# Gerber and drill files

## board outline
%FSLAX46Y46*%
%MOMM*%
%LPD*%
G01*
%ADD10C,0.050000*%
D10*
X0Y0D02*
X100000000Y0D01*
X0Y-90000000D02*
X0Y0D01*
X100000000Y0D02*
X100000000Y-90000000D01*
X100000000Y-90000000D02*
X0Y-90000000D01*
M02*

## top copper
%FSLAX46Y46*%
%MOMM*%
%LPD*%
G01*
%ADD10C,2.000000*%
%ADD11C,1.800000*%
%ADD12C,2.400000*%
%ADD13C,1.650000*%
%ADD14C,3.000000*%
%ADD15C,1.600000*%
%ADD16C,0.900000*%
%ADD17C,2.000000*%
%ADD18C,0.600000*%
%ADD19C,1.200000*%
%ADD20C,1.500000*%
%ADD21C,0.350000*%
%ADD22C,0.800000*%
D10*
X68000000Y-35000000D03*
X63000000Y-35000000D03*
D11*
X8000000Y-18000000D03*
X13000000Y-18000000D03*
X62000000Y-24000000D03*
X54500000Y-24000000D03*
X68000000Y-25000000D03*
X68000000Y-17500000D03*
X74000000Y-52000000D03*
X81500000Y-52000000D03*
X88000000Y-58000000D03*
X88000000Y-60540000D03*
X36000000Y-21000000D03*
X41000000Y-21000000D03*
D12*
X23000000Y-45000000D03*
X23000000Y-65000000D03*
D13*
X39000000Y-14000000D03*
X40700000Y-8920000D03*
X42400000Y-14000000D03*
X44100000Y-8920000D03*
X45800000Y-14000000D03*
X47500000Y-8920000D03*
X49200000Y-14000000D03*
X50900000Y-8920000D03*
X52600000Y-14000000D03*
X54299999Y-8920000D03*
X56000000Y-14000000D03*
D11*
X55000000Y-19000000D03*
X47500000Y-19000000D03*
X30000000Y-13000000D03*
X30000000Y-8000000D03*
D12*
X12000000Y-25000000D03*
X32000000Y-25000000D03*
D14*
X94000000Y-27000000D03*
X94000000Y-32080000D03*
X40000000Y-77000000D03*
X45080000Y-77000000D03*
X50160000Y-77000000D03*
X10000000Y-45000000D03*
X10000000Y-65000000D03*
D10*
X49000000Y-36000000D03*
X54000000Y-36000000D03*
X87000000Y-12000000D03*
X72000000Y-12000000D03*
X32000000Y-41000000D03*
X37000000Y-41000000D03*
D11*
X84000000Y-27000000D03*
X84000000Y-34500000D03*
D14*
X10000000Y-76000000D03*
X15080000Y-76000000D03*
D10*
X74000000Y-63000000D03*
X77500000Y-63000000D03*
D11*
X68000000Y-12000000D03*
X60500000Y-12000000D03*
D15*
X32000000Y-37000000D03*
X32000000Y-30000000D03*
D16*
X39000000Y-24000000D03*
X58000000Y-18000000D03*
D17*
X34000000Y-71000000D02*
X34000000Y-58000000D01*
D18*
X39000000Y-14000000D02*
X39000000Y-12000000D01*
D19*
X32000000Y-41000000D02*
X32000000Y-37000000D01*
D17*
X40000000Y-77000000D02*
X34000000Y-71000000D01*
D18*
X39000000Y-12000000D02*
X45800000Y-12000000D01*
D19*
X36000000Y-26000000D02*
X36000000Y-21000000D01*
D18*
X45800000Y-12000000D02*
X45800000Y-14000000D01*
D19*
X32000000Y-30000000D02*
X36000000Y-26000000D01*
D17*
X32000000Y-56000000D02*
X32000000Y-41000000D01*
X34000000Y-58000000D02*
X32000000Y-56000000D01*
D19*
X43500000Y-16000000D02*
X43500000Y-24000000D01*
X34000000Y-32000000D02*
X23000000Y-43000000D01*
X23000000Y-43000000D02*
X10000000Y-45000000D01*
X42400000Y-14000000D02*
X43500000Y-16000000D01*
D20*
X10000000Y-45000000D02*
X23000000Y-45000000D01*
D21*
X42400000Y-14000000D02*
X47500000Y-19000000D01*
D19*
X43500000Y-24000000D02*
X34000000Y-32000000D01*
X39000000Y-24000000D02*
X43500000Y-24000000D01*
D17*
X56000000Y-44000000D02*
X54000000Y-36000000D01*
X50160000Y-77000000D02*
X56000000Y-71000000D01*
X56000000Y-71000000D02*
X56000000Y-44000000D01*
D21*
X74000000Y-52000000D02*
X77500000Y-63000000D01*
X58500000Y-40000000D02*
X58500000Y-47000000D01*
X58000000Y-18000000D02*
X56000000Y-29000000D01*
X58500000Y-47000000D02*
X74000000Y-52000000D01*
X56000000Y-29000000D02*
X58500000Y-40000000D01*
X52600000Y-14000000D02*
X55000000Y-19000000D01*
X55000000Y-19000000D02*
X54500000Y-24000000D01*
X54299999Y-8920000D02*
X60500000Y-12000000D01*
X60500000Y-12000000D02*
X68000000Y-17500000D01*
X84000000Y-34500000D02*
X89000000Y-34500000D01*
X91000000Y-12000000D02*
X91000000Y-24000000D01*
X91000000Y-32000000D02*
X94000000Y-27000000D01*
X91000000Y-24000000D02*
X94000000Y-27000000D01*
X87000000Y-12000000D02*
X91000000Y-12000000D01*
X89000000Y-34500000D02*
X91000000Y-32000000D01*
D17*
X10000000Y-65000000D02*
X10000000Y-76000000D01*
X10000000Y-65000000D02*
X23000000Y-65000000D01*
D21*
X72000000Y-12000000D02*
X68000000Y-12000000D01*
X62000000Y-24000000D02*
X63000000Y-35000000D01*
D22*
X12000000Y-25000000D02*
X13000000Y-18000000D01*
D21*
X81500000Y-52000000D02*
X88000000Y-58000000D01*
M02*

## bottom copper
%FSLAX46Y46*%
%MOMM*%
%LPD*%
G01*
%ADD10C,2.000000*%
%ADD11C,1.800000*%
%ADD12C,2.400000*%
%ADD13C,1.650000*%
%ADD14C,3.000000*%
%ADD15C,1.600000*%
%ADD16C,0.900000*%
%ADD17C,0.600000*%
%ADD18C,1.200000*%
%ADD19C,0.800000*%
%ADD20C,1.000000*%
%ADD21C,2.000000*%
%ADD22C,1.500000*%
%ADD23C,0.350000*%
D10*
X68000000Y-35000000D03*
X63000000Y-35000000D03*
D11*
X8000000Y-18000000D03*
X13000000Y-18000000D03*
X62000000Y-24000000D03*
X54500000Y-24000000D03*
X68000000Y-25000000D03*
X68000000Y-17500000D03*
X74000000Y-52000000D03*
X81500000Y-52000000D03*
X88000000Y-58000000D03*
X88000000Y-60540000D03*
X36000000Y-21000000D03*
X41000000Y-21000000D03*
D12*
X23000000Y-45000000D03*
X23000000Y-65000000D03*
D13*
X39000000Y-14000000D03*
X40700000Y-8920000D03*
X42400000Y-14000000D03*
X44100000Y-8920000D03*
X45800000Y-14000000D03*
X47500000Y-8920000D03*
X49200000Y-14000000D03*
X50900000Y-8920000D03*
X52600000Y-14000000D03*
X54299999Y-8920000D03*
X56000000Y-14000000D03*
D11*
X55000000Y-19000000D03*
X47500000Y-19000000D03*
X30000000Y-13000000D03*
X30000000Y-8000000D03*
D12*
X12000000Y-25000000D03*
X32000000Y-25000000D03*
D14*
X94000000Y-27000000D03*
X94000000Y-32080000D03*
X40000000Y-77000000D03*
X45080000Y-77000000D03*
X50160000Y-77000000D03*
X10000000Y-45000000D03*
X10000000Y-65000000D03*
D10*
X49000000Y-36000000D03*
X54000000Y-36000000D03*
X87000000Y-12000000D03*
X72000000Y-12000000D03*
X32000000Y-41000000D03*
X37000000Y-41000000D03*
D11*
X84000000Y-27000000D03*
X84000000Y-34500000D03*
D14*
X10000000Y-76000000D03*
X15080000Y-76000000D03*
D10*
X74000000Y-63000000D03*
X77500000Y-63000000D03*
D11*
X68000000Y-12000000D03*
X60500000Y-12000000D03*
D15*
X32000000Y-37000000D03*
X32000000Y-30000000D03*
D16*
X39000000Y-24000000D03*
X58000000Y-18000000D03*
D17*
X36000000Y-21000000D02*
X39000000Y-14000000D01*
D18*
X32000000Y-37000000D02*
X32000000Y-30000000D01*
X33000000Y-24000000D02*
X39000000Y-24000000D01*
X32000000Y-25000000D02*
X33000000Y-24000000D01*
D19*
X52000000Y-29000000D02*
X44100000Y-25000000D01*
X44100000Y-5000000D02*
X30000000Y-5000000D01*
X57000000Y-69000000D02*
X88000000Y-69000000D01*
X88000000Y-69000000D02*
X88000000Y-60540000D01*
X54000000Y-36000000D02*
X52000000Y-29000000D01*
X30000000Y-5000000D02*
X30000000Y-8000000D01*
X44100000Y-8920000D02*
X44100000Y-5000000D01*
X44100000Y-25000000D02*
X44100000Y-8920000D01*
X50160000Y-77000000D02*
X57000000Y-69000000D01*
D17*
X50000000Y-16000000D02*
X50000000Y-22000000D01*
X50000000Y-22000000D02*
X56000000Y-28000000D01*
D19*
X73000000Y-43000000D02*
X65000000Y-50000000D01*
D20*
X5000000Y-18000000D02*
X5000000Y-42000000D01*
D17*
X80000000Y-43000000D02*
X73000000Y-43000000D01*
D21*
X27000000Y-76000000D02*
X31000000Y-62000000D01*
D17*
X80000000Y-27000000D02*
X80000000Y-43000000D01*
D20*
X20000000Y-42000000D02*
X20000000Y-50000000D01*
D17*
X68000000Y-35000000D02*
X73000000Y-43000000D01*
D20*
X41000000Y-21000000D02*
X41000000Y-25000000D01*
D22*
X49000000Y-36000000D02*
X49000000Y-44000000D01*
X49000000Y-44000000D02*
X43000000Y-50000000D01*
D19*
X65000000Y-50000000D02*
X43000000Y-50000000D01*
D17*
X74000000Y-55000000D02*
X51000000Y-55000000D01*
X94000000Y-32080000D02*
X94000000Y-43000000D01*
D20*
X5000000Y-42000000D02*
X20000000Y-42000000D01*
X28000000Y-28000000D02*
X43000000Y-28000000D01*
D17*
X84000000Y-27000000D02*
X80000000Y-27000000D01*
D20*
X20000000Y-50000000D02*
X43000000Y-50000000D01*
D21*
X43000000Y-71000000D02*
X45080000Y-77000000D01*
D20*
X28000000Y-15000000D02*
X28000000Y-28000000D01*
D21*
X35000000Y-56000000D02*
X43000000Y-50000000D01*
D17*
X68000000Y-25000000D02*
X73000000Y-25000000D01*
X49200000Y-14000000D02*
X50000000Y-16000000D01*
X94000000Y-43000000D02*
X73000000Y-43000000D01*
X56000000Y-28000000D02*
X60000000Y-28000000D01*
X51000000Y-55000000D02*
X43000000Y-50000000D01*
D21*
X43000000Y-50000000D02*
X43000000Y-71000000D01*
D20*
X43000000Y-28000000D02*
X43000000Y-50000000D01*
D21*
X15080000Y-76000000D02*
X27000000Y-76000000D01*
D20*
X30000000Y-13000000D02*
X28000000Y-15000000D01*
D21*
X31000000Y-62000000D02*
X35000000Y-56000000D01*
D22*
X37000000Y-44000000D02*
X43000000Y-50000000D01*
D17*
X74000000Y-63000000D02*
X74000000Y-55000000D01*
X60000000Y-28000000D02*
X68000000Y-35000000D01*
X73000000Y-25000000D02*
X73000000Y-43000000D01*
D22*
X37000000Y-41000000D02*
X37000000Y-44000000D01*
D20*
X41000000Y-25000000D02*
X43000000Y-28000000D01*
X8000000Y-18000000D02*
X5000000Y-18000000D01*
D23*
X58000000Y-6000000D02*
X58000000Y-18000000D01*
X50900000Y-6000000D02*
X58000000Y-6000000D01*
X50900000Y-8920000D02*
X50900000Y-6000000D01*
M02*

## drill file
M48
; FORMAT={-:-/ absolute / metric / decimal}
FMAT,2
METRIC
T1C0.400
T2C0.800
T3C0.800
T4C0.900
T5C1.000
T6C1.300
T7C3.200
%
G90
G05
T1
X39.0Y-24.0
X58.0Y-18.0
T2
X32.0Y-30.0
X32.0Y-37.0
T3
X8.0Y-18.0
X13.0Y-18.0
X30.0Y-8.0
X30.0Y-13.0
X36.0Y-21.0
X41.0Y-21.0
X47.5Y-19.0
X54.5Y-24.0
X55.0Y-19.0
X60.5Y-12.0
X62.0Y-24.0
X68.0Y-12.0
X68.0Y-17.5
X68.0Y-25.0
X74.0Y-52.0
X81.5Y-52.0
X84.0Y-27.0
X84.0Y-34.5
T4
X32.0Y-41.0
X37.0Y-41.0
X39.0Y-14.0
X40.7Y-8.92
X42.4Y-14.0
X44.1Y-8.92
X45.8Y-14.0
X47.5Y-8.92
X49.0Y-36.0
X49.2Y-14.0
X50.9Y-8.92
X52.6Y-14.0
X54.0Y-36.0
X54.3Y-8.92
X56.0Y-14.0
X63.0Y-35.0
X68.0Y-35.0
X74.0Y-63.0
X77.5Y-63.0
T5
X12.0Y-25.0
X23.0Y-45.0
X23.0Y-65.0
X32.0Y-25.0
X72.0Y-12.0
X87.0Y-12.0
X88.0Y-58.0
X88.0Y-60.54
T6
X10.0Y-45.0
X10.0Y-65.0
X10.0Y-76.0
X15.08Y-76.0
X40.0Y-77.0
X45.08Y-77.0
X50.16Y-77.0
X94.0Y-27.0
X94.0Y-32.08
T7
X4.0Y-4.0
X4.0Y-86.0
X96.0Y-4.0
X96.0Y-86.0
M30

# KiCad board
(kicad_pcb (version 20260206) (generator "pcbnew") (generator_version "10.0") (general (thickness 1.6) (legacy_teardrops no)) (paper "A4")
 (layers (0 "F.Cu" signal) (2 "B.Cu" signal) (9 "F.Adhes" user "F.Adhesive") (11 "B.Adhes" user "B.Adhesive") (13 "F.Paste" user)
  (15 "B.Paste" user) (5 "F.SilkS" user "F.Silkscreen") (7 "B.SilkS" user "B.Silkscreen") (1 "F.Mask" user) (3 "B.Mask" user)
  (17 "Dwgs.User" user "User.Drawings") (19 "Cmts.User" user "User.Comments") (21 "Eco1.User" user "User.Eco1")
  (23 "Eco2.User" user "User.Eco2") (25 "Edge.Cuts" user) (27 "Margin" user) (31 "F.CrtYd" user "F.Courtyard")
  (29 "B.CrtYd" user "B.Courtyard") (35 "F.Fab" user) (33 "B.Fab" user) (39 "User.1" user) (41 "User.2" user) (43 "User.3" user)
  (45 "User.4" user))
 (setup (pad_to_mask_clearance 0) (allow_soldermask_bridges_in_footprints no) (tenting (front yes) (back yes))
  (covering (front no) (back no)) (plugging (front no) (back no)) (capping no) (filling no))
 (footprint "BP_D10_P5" (layer "F.Cu") (at 68 35 180)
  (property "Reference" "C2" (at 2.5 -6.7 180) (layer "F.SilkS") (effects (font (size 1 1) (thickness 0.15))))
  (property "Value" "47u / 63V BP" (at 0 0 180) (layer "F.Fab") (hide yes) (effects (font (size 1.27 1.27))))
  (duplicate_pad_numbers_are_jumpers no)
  (pad "1" thru_hole circle (at 0 0 180) (size 2 2) (drill 0.9) (layers "*.Cu" "*.Mask") (remove_unused_layers no) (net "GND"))
  (pad "2" thru_hole circle (at 5 0 180) (size 2 2) (drill 0.9) (layers "*.Cu" "*.Mask") (remove_unused_layers no) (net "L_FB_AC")))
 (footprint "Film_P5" (layer "F.Cu") (at 8 18)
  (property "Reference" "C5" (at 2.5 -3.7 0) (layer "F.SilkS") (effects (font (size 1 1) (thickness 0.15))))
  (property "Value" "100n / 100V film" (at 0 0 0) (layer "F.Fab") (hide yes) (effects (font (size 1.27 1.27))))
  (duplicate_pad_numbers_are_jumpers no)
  (pad "1" thru_hole circle (at 0 0) (size 1.8 1.8) (drill 0.8) (layers "*.Cu" "*.Mask") (remove_unused_layers no) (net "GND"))
  (pad "2" thru_hole circle (at 5 0) (size 1.8 1.8) (drill 0.8) (layers "*.Cu" "*.Mask") (remove_unused_layers no) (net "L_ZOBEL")))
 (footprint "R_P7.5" (layer "F.Cu") (at 62 24 180)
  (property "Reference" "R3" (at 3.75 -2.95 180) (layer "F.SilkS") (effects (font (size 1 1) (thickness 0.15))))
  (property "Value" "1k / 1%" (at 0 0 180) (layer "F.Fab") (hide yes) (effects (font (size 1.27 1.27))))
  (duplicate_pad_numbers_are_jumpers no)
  (pad "1" thru_hole circle (at 0 0 180) (size 1.8 1.8) (drill 0.8) (layers "*.Cu" "*.Mask") (remove_unused_layers no) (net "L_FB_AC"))
  (pad "2" thru_hole circle (at 7.5 0 180) (size 1.8 1.8) (drill 0.8) (layers "*.Cu" "*.Mask") (remove_unused_layers no) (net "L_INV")))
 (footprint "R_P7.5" (layer "F.Cu") (at 68 25 90)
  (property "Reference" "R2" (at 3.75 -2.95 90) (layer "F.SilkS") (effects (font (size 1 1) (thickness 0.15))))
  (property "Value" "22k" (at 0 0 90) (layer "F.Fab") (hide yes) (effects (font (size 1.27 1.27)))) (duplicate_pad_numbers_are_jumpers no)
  (pad "1" thru_hole circle (at 0 0 90) (size 1.8 1.8) (drill 0.8) (layers "*.Cu" "*.Mask") (remove_unused_layers no) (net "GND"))
  (pad "2" thru_hole circle (at 7.5 0 90) (size 1.8 1.8) (drill 0.8) (layers "*.Cu" "*.Mask") (remove_unused_layers no) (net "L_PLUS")))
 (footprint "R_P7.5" (layer "F.Cu") (at 74 52)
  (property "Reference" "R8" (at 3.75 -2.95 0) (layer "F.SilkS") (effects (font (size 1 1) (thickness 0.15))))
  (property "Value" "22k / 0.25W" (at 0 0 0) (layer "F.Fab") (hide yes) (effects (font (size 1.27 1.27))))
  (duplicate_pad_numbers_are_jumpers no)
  (pad "1" thru_hole circle (at 0 0) (size 1.8 1.8) (drill 0.8) (layers "*.Cu" "*.Mask") (remove_unused_layers no) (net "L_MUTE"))
  (pad "2" thru_hole circle (at 7.5 0) (size 1.8 1.8) (drill 0.8) (layers "*.Cu" "*.Mask") (remove_unused_layers no) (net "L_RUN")))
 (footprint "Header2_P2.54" (layer "F.Cu") (at 88 58 -90)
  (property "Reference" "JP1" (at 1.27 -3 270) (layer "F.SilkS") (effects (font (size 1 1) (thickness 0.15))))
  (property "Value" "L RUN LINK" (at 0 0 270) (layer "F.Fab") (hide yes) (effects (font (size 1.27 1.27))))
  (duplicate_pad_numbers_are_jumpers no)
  (pad "1" thru_hole circle (at 0 0 270) (size 1.8 1.8) (drill 1) (layers "*.Cu" "*.Mask") (remove_unused_layers no) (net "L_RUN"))
  (pad "2" thru_hole circle (at 2.54 0 270) (size 1.8 1.8) (drill 1) (layers "*.Cu" "*.Mask") (remove_unused_layers no) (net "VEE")))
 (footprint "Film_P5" (layer "F.Cu") (at 36 21)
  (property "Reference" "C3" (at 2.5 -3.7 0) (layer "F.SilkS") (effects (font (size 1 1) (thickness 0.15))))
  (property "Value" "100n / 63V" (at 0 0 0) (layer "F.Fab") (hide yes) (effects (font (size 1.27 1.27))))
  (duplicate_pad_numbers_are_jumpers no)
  (pad "1" thru_hole circle (at 0 0) (size 1.8 1.8) (drill 0.8) (layers "*.Cu" "*.Mask") (remove_unused_layers no) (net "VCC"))
  (pad "2" thru_hole circle (at 5 0) (size 1.8 1.8) (drill 0.8) (layers "*.Cu" "*.Mask") (remove_unused_layers no) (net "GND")))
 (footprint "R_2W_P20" (layer "F.Cu") (at 23 45 -90)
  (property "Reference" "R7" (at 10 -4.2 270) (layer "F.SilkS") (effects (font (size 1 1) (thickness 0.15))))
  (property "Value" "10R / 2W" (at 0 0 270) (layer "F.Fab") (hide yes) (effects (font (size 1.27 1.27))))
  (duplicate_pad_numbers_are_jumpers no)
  (pad "1" thru_hole circle (at 0 0 270) (size 2.4 2.4) (drill 1) (layers "*.Cu" "*.Mask") (remove_unused_layers no) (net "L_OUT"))
  (pad "2" thru_hole circle (at 20 0 270) (size 2.4 2.4) (drill 1) (layers "*.Cu" "*.Mask") (remove_unused_layers no) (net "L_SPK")))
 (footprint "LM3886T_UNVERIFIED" (layer "F.Cu") (at 39 14)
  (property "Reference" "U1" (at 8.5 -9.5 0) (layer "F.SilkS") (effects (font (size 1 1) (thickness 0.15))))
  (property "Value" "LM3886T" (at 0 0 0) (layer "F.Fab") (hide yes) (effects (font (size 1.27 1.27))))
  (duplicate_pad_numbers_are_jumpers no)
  (pad "1" thru_hole circle (at 0 0) (size 1.65 1.65) (drill 0.9) (layers "*.Cu" "*.Mask") (remove_unused_layers no) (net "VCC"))
  (pad "2" thru_hole circle (at 1.7 -5.08) (size 1.65 1.65) (drill 0.9) (layers "*.Cu" "*.Mask") (remove_unused_layers no)
   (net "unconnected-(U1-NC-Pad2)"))
  (pad "3" thru_hole circle (at 3.4 0) (size 1.65 1.65) (drill 0.9) (layers "*.Cu" "*.Mask") (remove_unused_layers no) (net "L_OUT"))
  (pad "4" thru_hole circle (at 5.1 -5.08) (size 1.65 1.65) (drill 0.9) (layers "*.Cu" "*.Mask") (remove_unused_layers no) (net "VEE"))
  (pad "5" thru_hole circle (at 6.8 0) (size 1.65 1.65) (drill 0.9) (layers "*.Cu" "*.Mask") (remove_unused_layers no) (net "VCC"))
  (pad "6" thru_hole circle (at 8.5 -5.08) (size 1.65 1.65) (drill 0.9) (layers "*.Cu" "*.Mask") (remove_unused_layers no)
   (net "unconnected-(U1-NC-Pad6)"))
  (pad "7" thru_hole circle (at 10.2 0) (size 1.65 1.65) (drill 0.9) (layers "*.Cu" "*.Mask") (remove_unused_layers no) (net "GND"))
  (pad "8" thru_hole circle (at 11.9 -5.08) (size 1.65 1.65) (drill 0.9) (layers "*.Cu" "*.Mask") (remove_unused_layers no) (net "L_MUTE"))
  (pad "9" thru_hole circle (at 13.6 0) (size 1.65 1.65) (drill 0.9) (layers "*.Cu" "*.Mask") (remove_unused_layers no) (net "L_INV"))
  (pad "10" thru_hole circle (at 15.299999 -5.08) (size 1.65 1.65) (drill 0.9) (layers "*.Cu" "*.Mask") (remove_unused_layers no)
   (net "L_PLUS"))
  (pad "11" thru_hole circle (at 17 0) (size 1.65 1.65) (drill 0.9) (layers "*.Cu" "*.Mask") (remove_unused_layers no)
   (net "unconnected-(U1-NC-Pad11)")))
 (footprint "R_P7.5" (layer "F.Cu") (at 55 19 180)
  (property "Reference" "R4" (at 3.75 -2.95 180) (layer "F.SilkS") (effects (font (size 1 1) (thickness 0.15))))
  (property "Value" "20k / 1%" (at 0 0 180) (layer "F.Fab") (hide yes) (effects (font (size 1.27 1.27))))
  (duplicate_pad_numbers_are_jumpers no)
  (pad "1" thru_hole circle (at 0 0 180) (size 1.8 1.8) (drill 0.8) (layers "*.Cu" "*.Mask") (remove_unused_layers no) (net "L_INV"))
  (pad "2" thru_hole circle (at 7.5 0 180) (size 1.8 1.8) (drill 0.8) (layers "*.Cu" "*.Mask") (remove_unused_layers no) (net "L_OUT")))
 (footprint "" (layer "F.Cu") (at 96 4)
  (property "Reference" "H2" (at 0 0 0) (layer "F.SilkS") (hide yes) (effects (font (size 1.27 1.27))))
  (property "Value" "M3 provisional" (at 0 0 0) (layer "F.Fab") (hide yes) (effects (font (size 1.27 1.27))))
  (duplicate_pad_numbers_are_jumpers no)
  (pad "" np_thru_hole circle (at 0 0) (size 3.2 3.2) (drill 3.2) (layers "*.Cu" "*.Mask")))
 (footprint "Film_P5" (layer "F.Cu") (at 30 13 90)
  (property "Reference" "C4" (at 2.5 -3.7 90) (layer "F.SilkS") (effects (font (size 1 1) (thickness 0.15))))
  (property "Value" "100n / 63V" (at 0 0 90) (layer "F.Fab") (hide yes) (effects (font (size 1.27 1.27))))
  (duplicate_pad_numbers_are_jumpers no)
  (pad "1" thru_hole circle (at 0 0 90) (size 1.8 1.8) (drill 0.8) (layers "*.Cu" "*.Mask") (remove_unused_layers no) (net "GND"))
  (pad "2" thru_hole circle (at 5 0 90) (size 1.8 1.8) (drill 0.8) (layers "*.Cu" "*.Mask") (remove_unused_layers no) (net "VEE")))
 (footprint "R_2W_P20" (layer "F.Cu") (at 12 25)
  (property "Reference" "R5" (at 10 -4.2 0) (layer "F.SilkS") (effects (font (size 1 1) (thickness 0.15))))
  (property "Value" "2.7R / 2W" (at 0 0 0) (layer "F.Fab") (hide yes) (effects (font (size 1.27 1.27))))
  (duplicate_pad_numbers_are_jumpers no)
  (pad "1" thru_hole circle (at 0 0) (size 2.4 2.4) (drill 1) (layers "*.Cu" "*.Mask") (remove_unused_layers no) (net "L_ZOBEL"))
  (pad "2" thru_hole circle (at 20 0) (size 2.4 2.4) (drill 1) (layers "*.Cu" "*.Mask") (remove_unused_layers no) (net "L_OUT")))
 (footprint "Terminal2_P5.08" (layer "F.Cu") (at 94 27 -90)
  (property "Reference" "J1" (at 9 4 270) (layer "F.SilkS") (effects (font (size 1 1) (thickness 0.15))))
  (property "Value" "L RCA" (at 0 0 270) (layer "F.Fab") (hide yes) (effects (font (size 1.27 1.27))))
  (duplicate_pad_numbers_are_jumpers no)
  (pad "1" thru_hole circle (at 0 0 270) (size 3 3) (drill 1.3) (layers "*.Cu" "*.Mask") (remove_unused_layers no) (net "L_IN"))
  (pad "2" thru_hole circle (at 5.08 0 270) (size 3 3) (drill 1.3) (layers "*.Cu" "*.Mask") (remove_unused_layers no) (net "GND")))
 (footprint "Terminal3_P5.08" (layer "F.Cu") (at 40 77)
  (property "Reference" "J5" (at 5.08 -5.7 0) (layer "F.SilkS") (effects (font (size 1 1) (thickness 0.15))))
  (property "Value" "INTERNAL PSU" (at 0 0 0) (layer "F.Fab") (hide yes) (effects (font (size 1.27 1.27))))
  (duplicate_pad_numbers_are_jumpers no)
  (pad "1" thru_hole circle (at 0 0) (size 3 3) (drill 1.3) (layers "*.Cu" "*.Mask") (remove_unused_layers no) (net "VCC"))
  (pad "2" thru_hole circle (at 5.08 0) (size 3 3) (drill 1.3) (layers "*.Cu" "*.Mask") (remove_unused_layers no) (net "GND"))
  (pad "3" thru_hole circle (at 10.16 0) (size 3 3) (drill 1.3) (layers "*.Cu" "*.Mask") (remove_unused_layers no) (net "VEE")))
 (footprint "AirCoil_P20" (layer "F.Cu") (at 10 45 -90)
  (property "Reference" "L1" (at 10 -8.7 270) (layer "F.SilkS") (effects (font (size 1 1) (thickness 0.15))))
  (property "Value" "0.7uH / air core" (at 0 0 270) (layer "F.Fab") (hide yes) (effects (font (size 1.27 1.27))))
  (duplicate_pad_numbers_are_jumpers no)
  (pad "1" thru_hole circle (at 0 0 270) (size 3 3) (drill 1.3) (layers "*.Cu" "*.Mask") (remove_unused_layers no) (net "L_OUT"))
  (pad "2" thru_hole circle (at 20 0 270) (size 3 3) (drill 1.3) (layers "*.Cu" "*.Mask") (remove_unused_layers no) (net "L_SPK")))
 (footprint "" (layer "F.Cu") (at 96 86)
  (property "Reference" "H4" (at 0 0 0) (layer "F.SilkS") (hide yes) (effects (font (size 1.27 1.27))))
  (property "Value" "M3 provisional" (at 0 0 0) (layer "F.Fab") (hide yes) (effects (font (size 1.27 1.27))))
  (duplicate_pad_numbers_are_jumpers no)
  (pad "" np_thru_hole circle (at 0 0) (size 3.2 3.2) (drill 3.2) (layers "*.Cu" "*.Mask")))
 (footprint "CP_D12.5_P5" (layer "F.Cu") (at 49 36)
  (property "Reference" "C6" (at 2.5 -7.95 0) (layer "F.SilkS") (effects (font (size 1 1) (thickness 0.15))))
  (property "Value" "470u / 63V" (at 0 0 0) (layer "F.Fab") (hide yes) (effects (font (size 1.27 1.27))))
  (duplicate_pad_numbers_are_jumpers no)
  (pad "1" thru_hole circle (at 0 0) (size 2 2) (drill 0.9) (layers "*.Cu" "*.Mask") (remove_unused_layers no) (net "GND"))
  (pad "2" thru_hole circle (at 5 0) (size 2 2) (drill 0.9) (layers "*.Cu" "*.Mask") (remove_unused_layers no) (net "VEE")))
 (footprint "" (layer "F.Cu") (at 4 4)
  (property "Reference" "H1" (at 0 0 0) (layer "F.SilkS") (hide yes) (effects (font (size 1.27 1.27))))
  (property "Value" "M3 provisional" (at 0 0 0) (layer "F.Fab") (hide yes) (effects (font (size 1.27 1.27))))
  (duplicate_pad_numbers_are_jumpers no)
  (pad "" np_thru_hole circle (at 0 0) (size 3.2 3.2) (drill 3.2) (layers "*.Cu" "*.Mask")))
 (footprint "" (layer "F.Cu") (at 4 86)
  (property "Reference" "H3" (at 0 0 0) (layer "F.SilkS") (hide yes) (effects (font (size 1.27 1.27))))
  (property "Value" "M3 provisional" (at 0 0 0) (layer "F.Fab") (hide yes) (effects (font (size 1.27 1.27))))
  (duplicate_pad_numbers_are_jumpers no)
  (pad "" np_thru_hole circle (at 0 0) (size 3.2 3.2) (drill 3.2) (layers "*.Cu" "*.Mask")))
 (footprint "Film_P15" (layer "F.Cu") (at 87 12 180)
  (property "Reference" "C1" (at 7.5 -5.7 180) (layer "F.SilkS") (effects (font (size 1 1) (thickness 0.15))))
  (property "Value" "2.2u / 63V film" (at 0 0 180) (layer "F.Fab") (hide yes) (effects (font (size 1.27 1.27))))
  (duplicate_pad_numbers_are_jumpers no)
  (pad "1" thru_hole circle (at 0 0 180) (size 2 2) (drill 1) (layers "*.Cu" "*.Mask") (remove_unused_layers no) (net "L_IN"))
  (pad "2" thru_hole circle (at 15 0 180) (size 2 2) (drill 1) (layers "*.Cu" "*.Mask") (remove_unused_layers no) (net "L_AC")))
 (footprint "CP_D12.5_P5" (layer "F.Cu") (at 32 41)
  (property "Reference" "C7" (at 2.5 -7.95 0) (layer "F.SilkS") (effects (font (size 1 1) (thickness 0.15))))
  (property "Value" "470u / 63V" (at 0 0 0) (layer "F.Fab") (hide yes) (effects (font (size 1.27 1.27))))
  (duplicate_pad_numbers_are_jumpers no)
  (pad "1" thru_hole circle (at 0 0) (size 2 2) (drill 0.9) (layers "*.Cu" "*.Mask") (remove_unused_layers no) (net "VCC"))
  (pad "2" thru_hole circle (at 5 0) (size 2 2) (drill 0.9) (layers "*.Cu" "*.Mask") (remove_unused_layers no) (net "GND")))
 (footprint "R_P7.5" (layer "F.Cu") (at 84 27 -90)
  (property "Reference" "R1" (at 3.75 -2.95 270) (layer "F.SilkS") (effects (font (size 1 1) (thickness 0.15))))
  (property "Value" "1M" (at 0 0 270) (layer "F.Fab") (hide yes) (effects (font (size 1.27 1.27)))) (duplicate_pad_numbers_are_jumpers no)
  (pad "1" thru_hole circle (at 0 0 270) (size 1.8 1.8) (drill 0.8) (layers "*.Cu" "*.Mask") (remove_unused_layers no) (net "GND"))
  (pad "2" thru_hole circle (at 7.5 0 270) (size 1.8 1.8) (drill 0.8) (layers "*.Cu" "*.Mask") (remove_unused_layers no) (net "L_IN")))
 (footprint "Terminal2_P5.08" (layer "F.Cu") (at 10 76)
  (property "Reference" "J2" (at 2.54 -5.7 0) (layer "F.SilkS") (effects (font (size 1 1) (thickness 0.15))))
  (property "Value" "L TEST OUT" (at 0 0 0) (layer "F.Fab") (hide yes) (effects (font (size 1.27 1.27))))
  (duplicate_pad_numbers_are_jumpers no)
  (pad "1" thru_hole circle (at 0 0) (size 3 3) (drill 1.3) (layers "*.Cu" "*.Mask") (remove_unused_layers no) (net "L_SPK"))
  (pad "2" thru_hole circle (at 5.08 0) (size 3 3) (drill 1.3) (layers "*.Cu" "*.Mask") (remove_unused_layers no) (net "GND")))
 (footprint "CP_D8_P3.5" (layer "F.Cu") (at 74 63)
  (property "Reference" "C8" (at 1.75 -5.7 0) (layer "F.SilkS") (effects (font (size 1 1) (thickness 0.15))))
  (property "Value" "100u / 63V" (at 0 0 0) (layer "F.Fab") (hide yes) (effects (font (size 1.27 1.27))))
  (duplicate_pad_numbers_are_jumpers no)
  (pad "1" thru_hole circle (at 0 0) (size 2 2) (drill 0.9) (layers "*.Cu" "*.Mask") (remove_unused_layers no) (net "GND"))
  (pad "2" thru_hole circle (at 3.5 0) (size 2 2) (drill 0.9) (layers "*.Cu" "*.Mask") (remove_unused_layers no) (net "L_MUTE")))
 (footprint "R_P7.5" (layer "F.Cu") (at 68 12 180)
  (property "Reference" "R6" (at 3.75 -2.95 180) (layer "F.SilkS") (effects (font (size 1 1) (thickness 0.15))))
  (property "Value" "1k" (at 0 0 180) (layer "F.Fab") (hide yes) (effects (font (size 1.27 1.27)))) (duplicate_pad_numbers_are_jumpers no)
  (pad "1" thru_hole circle (at 0 0 180) (size 1.8 1.8) (drill 0.8) (layers "*.Cu" "*.Mask") (remove_unused_layers no) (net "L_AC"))
  (pad "2" thru_hole circle (at 7.5 0 180) (size 1.8 1.8) (drill 0.8) (layers "*.Cu" "*.Mask") (remove_unused_layers no) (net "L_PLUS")))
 (gr_line (start 0 0) (end 100 0) (stroke (width 0.05) (type default)) (layer "Edge.Cuts"))
 (gr_line (start 0 90) (end 0 0) (stroke (width 0.05) (type default)) (layer "Edge.Cuts"))
 (gr_line (start 100 0) (end 100 90) (stroke (width 0.05) (type default)) (layer "Edge.Cuts"))
 (gr_line (start 100 90) (end 0 90) (stroke (width 0.05) (type default)) (layer "Edge.Cuts"))
 (segment (start 34 71) (end 34 58) (width 2) (layer "F.Cu") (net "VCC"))
 (segment (start 39 14) (end 39 12) (width 0.6) (layer "F.Cu") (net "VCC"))
 (segment (start 32 41) (end 32 37) (width 1.2) (layer "F.Cu") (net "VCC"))
 (segment (start 40 77) (end 34 71) (width 2) (layer "F.Cu") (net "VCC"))
 (segment (start 39 12) (end 45.8 12) (width 0.6) (layer "F.Cu") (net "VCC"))
 (segment (start 36 26) (end 36 21) (width 1.2) (layer "F.Cu") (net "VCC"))
 (segment (start 45.8 12) (end 45.8 14) (width 0.6) (layer "F.Cu") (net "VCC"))
 (segment (start 32 30) (end 36 26) (width 1.2) (layer "F.Cu") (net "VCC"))
 (segment (start 32 56) (end 32 41) (width 2) (layer "F.Cu") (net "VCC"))
 (segment (start 34 58) (end 32 56) (width 2) (layer "F.Cu") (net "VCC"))
 (via (at 32 37) (size 1.6) (drill 0.8) (layers "F.Cu" "B.Cu") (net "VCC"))
 (via (at 32 30) (size 1.6) (drill 0.8) (layers "F.Cu" "B.Cu") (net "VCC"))
 (segment (start 36 21) (end 39 14) (width 0.6) (layer "B.Cu") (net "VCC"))
 (segment (start 32 37) (end 32 30) (width 1.2) (layer "B.Cu") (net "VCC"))
 (segment (start 43.5 16) (end 43.5 24) (width 1.2) (layer "F.Cu") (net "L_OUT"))
 (segment (start 34 32) (end 23 43) (width 1.2) (layer "F.Cu") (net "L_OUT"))
 (segment (start 23 43) (end 10 45) (width 1.2) (layer "F.Cu") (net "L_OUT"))
 (segment (start 42.4 14) (end 43.5 16) (width 1.2) (layer "F.Cu") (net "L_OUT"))
 (segment (start 10 45) (end 23 45) (width 1.5) (layer "F.Cu") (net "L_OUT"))
 (segment (start 42.4 14) (end 47.5 19) (width 0.35) (layer "F.Cu") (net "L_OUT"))
 (segment (start 43.5 24) (end 34 32) (width 1.2) (layer "F.Cu") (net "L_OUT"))
 (segment (start 39 24) (end 43.5 24) (width 1.2) (layer "F.Cu") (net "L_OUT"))
 (via (at 39 24) (size 0.9) (drill 0.4) (layers "F.Cu" "B.Cu") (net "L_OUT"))
 (segment (start 33 24) (end 39 24) (width 1.2) (layer "B.Cu") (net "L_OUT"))
 (segment (start 32 25) (end 33 24) (width 1.2) (layer "B.Cu") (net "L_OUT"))
 (segment (start 56 44) (end 54 36) (width 2) (layer "F.Cu") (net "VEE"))
 (segment (start 50.16 77) (end 56 71) (width 2) (layer "F.Cu") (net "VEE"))
 (segment (start 56 71) (end 56 44) (width 2) (layer "F.Cu") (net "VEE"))
 (segment (start 52 29) (end 44.1 25) (width 0.8) (layer "B.Cu") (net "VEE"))
 (segment (start 44.1 5) (end 30 5) (width 0.8) (layer "B.Cu") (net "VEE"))
 (segment (start 57 69) (end 88 69) (width 0.8) (layer "B.Cu") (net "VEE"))
 (segment (start 88 69) (end 88 60.54) (width 0.8) (layer "B.Cu") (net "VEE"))
 (segment (start 54 36) (end 52 29) (width 0.8) (layer "B.Cu") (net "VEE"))
 (segment (start 30 5) (end 30 8) (width 0.8) (layer "B.Cu") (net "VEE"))
 (segment (start 44.1 8.92) (end 44.1 5) (width 0.8) (layer "B.Cu") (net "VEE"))
 (segment (start 44.1 25) (end 44.1 8.92) (width 0.8) (layer "B.Cu") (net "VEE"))
 (segment (start 50.16 77) (end 57 69) (width 0.8) (layer "B.Cu") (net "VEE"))
 (segment (start 50 16) (end 50 22) (width 0.6) (layer "B.Cu") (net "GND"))
 (segment (start 50 22) (end 56 28) (width 0.6) (layer "B.Cu") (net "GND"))
 (segment (start 73 43) (end 65 50) (width 0.8) (layer "B.Cu") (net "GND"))
 (segment (start 5 18) (end 5 42) (width 1) (layer "B.Cu") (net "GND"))
 (segment (start 80 43) (end 73 43) (width 0.6) (layer "B.Cu") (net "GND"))
 (segment (start 27 76) (end 31 62) (width 2) (layer "B.Cu") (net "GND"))
 (segment (start 80 27) (end 80 43) (width 0.6) (layer "B.Cu") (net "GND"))
 (segment (start 20 42) (end 20 50) (width 1) (layer "B.Cu") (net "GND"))
 (segment (start 68 35) (end 73 43) (width 0.6) (layer "B.Cu") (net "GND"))
 (segment (start 41 21) (end 41 25) (width 1) (layer "B.Cu") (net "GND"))
 (segment (start 49 36) (end 49 44) (width 1.5) (layer "B.Cu") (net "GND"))
 (segment (start 49 44) (end 43 50) (width 1.5) (layer "B.Cu") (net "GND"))
 (segment (start 65 50) (end 43 50) (width 0.8) (layer "B.Cu") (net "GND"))
 (segment (start 74 55) (end 51 55) (width 0.6) (layer "B.Cu") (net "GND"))
 (segment (start 94 32.08) (end 94 43) (width 0.6) (layer "B.Cu") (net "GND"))
 (segment (start 5 42) (end 20 42) (width 1) (layer "B.Cu") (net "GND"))
 (segment (start 28 28) (end 43 28) (width 1) (layer "B.Cu") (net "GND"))
 (segment (start 84 27) (end 80 27) (width 0.6) (layer "B.Cu") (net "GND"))
 (segment (start 20 50) (end 43 50) (width 1) (layer "B.Cu") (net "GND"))
 (segment (start 43 71) (end 45.08 77) (width 2) (layer "B.Cu") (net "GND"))
 (segment (start 28 15) (end 28 28) (width 1) (layer "B.Cu") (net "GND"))
 (segment (start 35 56) (end 43 50) (width 2) (layer "B.Cu") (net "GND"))
 (segment (start 68 25) (end 73 25) (width 0.6) (layer "B.Cu") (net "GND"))
 (segment (start 49.2 14) (end 50 16) (width 0.6) (layer "B.Cu") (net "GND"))
 (segment (start 94 43) (end 73 43) (width 0.6) (layer "B.Cu") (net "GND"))
 (segment (start 56 28) (end 60 28) (width 0.6) (layer "B.Cu") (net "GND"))
 (segment (start 51 55) (end 43 50) (width 0.6) (layer "B.Cu") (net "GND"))
 (segment (start 43 50) (end 43 71) (width 2) (layer "B.Cu") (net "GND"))
 (segment (start 43 28) (end 43 50) (width 1) (layer "B.Cu") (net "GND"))
 (segment (start 15.08 76) (end 27 76) (width 2) (layer "B.Cu") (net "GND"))
 (segment (start 30 13) (end 28 15) (width 1) (layer "B.Cu") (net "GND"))
 (segment (start 31 62) (end 35 56) (width 2) (layer "B.Cu") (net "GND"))
 (segment (start 37 44) (end 43 50) (width 1.5) (layer "B.Cu") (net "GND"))
 (segment (start 74 63) (end 74 55) (width 0.6) (layer "B.Cu") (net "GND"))
 (segment (start 60 28) (end 68 35) (width 0.6) (layer "B.Cu") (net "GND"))
 (segment (start 73 25) (end 73 43) (width 0.6) (layer "B.Cu") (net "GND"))
 (segment (start 37 41) (end 37 44) (width 1.5) (layer "B.Cu") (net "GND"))
 (segment (start 41 25) (end 43 28) (width 1) (layer "B.Cu") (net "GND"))
 (segment (start 8 18) (end 5 18) (width 1) (layer "B.Cu") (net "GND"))
 (segment (start 74 52) (end 77.5 63) (width 0.35) (layer "F.Cu") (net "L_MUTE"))
 (segment (start 58.5 40) (end 58.5 47) (width 0.35) (layer "F.Cu") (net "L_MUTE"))
 (segment (start 58 18) (end 56 29) (width 0.35) (layer "F.Cu") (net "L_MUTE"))
 (segment (start 58.5 47) (end 74 52) (width 0.35) (layer "F.Cu") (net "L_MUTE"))
 (segment (start 56 29) (end 58.5 40) (width 0.35) (layer "F.Cu") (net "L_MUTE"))
 (via (at 58 18) (size 0.9) (drill 0.4) (layers "F.Cu" "B.Cu") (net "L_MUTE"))
 (segment (start 58 6) (end 58 18) (width 0.35) (layer "B.Cu") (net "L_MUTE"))
 (segment (start 50.9 6) (end 58 6) (width 0.35) (layer "B.Cu") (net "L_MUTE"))
 (segment (start 50.9 8.92) (end 50.9 6) (width 0.35) (layer "B.Cu") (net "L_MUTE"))
 (segment (start 52.6 14) (end 55 19) (width 0.35) (layer "F.Cu") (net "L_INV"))
 (segment (start 55 19) (end 54.5 24) (width 0.35) (layer "F.Cu") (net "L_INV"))
 (segment (start 54.299999 8.92) (end 60.5 12) (width 0.35) (layer "F.Cu") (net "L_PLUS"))
 (segment (start 60.5 12) (end 68 17.5) (width 0.35) (layer "F.Cu") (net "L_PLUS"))
 (segment (start 84 34.5) (end 89 34.5) (width 0.35) (layer "F.Cu") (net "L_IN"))
 (segment (start 91 12) (end 91 24) (width 0.35) (layer "F.Cu") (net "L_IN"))
 (segment (start 91 32) (end 94 27) (width 0.35) (layer "F.Cu") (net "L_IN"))
 (segment (start 91 24) (end 94 27) (width 0.35) (layer "F.Cu") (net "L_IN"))
 (segment (start 87 12) (end 91 12) (width 0.35) (layer "F.Cu") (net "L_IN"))
 (segment (start 89 34.5) (end 91 32) (width 0.35) (layer "F.Cu") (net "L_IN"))
 (segment (start 10 65) (end 10 76) (width 2) (layer "F.Cu") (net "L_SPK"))
 (segment (start 10 65) (end 23 65) (width 2) (layer "F.Cu") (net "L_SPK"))
 (segment (start 72 12) (end 68 12) (width 0.35) (layer "F.Cu") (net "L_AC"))
 (segment (start 62 24) (end 63 35) (width 0.35) (layer "F.Cu") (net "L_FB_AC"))
 (segment (start 12 25) (end 13 18) (width 0.8) (layer "F.Cu") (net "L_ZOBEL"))
 (segment (start 81.5 52) (end 88 58) (width 0.35) (layer "F.Cu") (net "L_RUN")))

